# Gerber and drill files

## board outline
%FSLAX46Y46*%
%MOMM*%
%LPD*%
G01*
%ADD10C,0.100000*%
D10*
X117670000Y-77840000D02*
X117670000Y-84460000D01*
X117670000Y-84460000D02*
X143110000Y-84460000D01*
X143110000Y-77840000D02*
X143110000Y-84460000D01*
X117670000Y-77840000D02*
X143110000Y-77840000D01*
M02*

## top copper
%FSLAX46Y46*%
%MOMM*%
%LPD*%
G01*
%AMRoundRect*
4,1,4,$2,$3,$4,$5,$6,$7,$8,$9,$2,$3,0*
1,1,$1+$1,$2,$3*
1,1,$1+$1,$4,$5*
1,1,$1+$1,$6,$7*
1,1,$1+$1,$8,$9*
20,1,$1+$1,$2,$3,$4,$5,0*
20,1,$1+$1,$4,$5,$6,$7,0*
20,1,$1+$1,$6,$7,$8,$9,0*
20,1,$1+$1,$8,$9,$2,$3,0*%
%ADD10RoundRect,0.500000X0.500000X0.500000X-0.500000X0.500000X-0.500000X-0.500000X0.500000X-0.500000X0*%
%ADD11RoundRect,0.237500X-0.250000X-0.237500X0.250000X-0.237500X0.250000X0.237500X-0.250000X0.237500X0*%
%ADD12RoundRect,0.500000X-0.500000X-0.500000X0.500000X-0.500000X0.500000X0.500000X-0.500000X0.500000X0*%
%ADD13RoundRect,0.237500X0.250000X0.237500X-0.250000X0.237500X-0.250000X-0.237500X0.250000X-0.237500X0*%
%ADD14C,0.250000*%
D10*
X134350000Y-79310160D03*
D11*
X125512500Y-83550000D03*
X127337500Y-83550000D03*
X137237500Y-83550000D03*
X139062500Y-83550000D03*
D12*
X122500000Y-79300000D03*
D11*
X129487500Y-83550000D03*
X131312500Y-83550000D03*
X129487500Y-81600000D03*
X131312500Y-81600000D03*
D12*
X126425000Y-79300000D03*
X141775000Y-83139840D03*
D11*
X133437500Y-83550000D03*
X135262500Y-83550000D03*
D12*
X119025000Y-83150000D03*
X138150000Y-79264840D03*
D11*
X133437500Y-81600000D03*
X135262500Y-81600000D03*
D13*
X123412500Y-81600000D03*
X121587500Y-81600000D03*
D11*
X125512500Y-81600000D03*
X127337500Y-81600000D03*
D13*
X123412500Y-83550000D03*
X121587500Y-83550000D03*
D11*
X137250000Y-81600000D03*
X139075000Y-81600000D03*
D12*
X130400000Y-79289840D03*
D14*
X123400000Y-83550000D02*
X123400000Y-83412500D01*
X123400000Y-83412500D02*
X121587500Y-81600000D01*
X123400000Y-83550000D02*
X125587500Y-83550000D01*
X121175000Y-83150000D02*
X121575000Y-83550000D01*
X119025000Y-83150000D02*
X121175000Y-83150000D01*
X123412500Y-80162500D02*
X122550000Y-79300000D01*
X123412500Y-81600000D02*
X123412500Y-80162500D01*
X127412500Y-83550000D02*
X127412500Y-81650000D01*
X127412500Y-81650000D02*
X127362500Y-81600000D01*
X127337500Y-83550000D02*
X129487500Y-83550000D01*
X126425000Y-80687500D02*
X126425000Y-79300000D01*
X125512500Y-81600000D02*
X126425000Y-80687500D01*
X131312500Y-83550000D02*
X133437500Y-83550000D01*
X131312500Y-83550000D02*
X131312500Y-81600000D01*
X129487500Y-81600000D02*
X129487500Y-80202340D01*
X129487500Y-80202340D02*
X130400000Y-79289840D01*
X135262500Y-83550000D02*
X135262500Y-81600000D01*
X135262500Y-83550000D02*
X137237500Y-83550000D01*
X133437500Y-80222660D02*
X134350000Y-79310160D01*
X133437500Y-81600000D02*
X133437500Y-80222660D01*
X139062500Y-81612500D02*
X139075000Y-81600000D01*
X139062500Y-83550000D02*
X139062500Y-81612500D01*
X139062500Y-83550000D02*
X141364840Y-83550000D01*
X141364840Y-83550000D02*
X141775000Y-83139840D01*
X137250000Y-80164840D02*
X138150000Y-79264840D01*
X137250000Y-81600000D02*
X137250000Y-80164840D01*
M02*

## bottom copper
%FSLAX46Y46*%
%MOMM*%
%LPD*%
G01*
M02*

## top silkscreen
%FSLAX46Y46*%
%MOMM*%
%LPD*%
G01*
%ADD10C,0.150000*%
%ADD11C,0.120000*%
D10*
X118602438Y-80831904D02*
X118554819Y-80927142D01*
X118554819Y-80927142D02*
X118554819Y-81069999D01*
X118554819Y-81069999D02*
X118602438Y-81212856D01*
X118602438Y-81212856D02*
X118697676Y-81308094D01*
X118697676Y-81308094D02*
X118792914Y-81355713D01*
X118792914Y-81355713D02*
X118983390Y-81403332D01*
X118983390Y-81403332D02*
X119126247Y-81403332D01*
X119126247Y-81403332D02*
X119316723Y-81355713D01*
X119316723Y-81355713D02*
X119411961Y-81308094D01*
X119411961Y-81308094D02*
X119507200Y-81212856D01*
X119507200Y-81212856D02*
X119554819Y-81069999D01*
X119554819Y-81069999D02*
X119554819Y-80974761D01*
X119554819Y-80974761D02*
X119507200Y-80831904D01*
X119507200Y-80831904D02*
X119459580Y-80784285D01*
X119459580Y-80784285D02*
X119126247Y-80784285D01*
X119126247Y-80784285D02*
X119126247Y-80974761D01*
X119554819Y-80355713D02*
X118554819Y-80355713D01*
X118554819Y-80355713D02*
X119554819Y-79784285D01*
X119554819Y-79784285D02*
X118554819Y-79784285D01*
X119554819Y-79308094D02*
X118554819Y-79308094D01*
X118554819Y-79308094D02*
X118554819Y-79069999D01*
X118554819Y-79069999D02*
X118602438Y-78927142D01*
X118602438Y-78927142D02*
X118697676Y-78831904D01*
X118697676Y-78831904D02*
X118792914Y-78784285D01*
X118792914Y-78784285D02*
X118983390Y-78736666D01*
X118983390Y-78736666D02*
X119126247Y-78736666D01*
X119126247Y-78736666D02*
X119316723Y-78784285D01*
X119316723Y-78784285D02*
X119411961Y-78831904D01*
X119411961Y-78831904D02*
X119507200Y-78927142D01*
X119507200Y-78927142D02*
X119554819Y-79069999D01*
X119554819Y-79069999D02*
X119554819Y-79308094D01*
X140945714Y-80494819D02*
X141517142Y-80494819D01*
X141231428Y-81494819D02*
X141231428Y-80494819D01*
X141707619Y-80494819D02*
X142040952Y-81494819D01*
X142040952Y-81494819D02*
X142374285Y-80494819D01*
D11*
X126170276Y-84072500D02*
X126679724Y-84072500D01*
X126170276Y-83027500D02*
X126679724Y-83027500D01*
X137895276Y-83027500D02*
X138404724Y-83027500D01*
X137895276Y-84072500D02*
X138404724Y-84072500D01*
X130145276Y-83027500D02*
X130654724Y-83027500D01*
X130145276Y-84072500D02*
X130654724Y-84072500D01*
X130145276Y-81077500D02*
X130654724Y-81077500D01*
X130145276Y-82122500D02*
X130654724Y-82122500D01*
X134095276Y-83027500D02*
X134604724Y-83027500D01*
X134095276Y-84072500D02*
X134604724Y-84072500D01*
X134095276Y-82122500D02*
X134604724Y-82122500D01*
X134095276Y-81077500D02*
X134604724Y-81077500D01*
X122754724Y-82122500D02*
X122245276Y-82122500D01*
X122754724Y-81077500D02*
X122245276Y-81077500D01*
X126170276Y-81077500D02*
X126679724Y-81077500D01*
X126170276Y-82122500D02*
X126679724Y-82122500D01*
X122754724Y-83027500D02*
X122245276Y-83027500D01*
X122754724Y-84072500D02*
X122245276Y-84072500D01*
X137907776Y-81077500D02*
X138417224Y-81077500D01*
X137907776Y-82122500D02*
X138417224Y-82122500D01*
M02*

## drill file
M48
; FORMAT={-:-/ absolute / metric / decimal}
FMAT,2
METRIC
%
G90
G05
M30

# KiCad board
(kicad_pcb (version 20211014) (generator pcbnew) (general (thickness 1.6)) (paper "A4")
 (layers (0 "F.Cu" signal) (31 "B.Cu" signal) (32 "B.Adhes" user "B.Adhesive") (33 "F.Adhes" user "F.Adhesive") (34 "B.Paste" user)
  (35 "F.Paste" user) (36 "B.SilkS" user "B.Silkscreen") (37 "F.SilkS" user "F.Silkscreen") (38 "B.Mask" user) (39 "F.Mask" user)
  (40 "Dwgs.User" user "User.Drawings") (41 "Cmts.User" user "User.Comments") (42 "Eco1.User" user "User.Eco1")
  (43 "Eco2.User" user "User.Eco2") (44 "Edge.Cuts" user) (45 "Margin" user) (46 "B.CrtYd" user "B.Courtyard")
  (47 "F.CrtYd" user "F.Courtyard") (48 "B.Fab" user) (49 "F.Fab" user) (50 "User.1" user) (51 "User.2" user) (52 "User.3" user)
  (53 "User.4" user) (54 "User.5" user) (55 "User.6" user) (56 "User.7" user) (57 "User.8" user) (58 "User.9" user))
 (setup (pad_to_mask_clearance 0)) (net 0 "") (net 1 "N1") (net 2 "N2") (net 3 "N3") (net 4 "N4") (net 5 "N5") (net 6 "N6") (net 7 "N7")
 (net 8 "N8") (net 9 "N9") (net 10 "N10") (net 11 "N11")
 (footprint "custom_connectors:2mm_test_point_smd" (layer "F.Cu") (at 134.35 79.3 180)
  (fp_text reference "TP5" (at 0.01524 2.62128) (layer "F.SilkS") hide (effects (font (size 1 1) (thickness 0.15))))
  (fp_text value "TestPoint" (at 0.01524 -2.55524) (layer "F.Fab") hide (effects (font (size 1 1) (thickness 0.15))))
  (pad "1" smd roundrect locked (at 0 -0.01016 180) (size 2 2) (layers "F.Cu" "F.Paste" "F.Mask") (roundrect_rratio 0.25) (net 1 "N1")))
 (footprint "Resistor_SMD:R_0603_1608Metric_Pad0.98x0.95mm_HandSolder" (layer "F.Cu") (at 126.425 83.55)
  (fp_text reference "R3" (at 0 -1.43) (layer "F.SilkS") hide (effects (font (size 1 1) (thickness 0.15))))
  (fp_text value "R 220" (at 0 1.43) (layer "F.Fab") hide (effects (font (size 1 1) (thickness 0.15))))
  (fp_line (start -0.254724 0.5225) (end 0.254724 0.5225) (layer "F.SilkS") (width 0.12))
  (fp_line (start -0.254724 -0.5225) (end 0.254724 -0.5225) (layer "F.SilkS") (width 0.12))
  (pad "1" smd roundrect (at -0.9125 0) (size 0.975 0.95) (layers "F.Cu" "F.Paste" "F.Mask") (roundrect_rratio 0.25) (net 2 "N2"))
  (pad "2" smd roundrect (at 0.9125 0) (size 0.975 0.95) (layers "F.Cu" "F.Paste" "F.Mask") (roundrect_rratio 0.25) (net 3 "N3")))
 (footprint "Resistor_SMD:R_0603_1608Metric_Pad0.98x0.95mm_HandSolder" (layer "F.Cu") (at 138.15 83.55)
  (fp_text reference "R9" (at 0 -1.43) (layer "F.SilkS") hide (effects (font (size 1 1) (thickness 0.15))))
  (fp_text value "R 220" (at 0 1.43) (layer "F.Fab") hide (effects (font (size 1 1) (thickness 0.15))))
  (fp_line (start -0.254724 -0.5225) (end 0.254724 -0.5225) (layer "F.SilkS") (width 0.12))
  (fp_line (start -0.254724 0.5225) (end 0.254724 0.5225) (layer "F.SilkS") (width 0.12))
  (pad "1" smd roundrect (at -0.9125 0) (size 0.975 0.95) (layers "F.Cu" "F.Paste" "F.Mask") (roundrect_rratio 0.25) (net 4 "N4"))
  (pad "2" smd roundrect (at 0.9125 0) (size 0.975 0.95) (layers "F.Cu" "F.Paste" "F.Mask") (roundrect_rratio 0.25) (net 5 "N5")))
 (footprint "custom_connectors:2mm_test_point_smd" (layer "F.Cu") (at 122.5 79.31016)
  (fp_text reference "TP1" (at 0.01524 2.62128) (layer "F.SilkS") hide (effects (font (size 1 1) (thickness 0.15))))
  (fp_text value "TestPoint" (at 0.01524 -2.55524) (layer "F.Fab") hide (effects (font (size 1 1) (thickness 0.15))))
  (pad "1" smd roundrect locked (at 0 -0.01016) (size 2 2) (layers "F.Cu" "F.Paste" "F.Mask") (roundrect_rratio 0.25) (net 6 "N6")))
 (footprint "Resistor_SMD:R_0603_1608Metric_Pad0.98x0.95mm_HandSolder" (layer "F.Cu") (at 130.4 83.55)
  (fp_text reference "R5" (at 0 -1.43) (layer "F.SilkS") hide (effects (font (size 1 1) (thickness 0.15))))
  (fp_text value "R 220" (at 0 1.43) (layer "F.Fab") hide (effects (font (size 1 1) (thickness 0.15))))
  (fp_line (start -0.254724 -0.5225) (end 0.254724 -0.5225) (layer "F.SilkS") (width 0.12))
  (fp_line (start -0.254724 0.5225) (end 0.254724 0.5225) (layer "F.SilkS") (width 0.12))
  (pad "1" smd roundrect (at -0.9125 0) (size 0.975 0.95) (layers "F.Cu" "F.Paste" "F.Mask") (roundrect_rratio 0.25) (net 3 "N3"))
  (pad "2" smd roundrect (at 0.9125 0) (size 0.975 0.95) (layers "F.Cu" "F.Paste" "F.Mask") (roundrect_rratio 0.25) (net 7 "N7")))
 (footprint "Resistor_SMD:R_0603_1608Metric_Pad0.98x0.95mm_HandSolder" (layer "F.Cu") (at 130.4 81.6)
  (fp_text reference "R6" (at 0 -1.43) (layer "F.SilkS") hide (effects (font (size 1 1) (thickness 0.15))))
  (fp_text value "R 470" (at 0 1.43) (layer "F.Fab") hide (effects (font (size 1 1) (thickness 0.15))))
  (fp_line (start -0.254724 -0.5225) (end 0.254724 -0.5225) (layer "F.SilkS") (width 0.12))
  (fp_line (start -0.254724 0.5225) (end 0.254724 0.5225) (layer "F.SilkS") (width 0.12))
  (pad "1" smd roundrect (at -0.9125 0) (size 0.975 0.95) (layers "F.Cu" "F.Paste" "F.Mask") (roundrect_rratio 0.25) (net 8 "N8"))
  (pad "2" smd roundrect (at 0.9125 0) (size 0.975 0.95) (layers "F.Cu" "F.Paste" "F.Mask") (roundrect_rratio 0.25) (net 7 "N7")))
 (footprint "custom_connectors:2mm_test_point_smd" (layer "F.Cu") (at 126.425 79.31016)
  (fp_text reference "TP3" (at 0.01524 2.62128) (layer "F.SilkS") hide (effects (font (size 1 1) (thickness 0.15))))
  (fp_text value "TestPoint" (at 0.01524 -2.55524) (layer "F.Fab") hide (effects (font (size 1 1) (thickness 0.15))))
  (pad "1" smd roundrect locked (at 0 -0.01016) (size 2 2) (layers "F.Cu" "F.Paste" "F.Mask") (roundrect_rratio 0.25) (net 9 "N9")))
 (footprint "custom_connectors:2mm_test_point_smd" (layer "F.Cu") (at 141.775 83.15)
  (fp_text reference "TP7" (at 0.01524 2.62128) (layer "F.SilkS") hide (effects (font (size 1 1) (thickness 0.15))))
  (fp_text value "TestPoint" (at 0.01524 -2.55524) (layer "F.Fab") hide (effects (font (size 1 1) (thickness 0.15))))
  (pad "1" smd roundrect locked (at 0 -0.01016) (size 2 2) (layers "F.Cu" "F.Paste" "F.Mask") (roundrect_rratio 0.25) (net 5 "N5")))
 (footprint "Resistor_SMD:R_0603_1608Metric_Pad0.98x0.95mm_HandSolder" (layer "F.Cu") (at 134.35 83.55)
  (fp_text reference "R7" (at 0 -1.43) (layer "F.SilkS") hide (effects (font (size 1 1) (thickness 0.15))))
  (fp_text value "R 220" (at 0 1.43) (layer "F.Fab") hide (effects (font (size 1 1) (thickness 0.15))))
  (fp_line (start -0.254724 -0.5225) (end 0.254724 -0.5225) (layer "F.SilkS") (width 0.12))
  (fp_line (start -0.254724 0.5225) (end 0.254724 0.5225) (layer "F.SilkS") (width 0.12))
  (pad "1" smd roundrect (at -0.9125 0) (size 0.975 0.95) (layers "F.Cu" "F.Paste" "F.Mask") (roundrect_rratio 0.25) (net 7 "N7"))
  (pad "2" smd roundrect (at 0.9125 0) (size 0.975 0.95) (layers "F.Cu" "F.Paste" "F.Mask") (roundrect_rratio 0.25) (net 4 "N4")))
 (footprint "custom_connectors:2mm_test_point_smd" (layer "F.Cu") (at 119.025 83.16016)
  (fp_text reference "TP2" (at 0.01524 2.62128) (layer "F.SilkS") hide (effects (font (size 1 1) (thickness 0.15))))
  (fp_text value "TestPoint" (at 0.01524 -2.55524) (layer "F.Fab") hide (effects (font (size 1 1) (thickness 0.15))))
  (pad "1" smd roundrect locked (at 0 -0.01016) (size 2 2) (layers "F.Cu" "F.Paste" "F.Mask") (roundrect_rratio 0.25) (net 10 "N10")))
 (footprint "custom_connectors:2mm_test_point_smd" (layer "F.Cu") (at 138.15 79.275)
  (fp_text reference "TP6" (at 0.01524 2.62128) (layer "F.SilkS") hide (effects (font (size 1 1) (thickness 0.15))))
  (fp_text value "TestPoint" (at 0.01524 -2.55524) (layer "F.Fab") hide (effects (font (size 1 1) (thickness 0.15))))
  (pad "1" smd roundrect locked (at 0 -0.01016) (size 2 2) (layers "F.Cu" "F.Paste" "F.Mask") (roundrect_rratio 0.25) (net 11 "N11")))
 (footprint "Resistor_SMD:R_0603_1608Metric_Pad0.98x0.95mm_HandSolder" (layer "F.Cu") (at 134.35 81.6)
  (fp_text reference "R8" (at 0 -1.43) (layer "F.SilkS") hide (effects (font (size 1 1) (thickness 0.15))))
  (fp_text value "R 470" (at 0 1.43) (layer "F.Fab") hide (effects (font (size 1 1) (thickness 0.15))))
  (fp_line (start -0.254724 0.5225) (end 0.254724 0.5225) (layer "F.SilkS") (width 0.12))
  (fp_line (start -0.254724 -0.5225) (end 0.254724 -0.5225) (layer "F.SilkS") (width 0.12))
  (pad "1" smd roundrect (at -0.9125 0) (size 0.975 0.95) (layers "F.Cu" "F.Paste" "F.Mask") (roundrect_rratio 0.25) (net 1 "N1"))
  (pad "2" smd roundrect (at 0.9125 0) (size 0.975 0.95) (layers "F.Cu" "F.Paste" "F.Mask") (roundrect_rratio 0.25) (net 4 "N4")))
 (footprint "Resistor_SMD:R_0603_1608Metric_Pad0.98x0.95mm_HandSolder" (layer "F.Cu") (at 122.5 81.6 180)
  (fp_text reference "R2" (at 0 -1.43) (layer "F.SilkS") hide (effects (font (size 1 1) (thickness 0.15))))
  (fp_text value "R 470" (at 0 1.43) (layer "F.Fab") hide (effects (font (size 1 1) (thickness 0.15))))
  (fp_line (start -0.254724 -0.5225) (end 0.254724 -0.5225) (layer "F.SilkS") (width 0.12))
  (fp_line (start -0.254724 0.5225) (end 0.254724 0.5225) (layer "F.SilkS") (width 0.12))
  (pad "1" smd roundrect (at -0.9125 0 180) (size 0.975 0.95) (layers "F.Cu" "F.Paste" "F.Mask") (roundrect_rratio 0.25) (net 6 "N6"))
  (pad "2" smd roundrect (at 0.9125 0 180) (size 0.975 0.95) (layers "F.Cu" "F.Paste" "F.Mask") (roundrect_rratio 0.25) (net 2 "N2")))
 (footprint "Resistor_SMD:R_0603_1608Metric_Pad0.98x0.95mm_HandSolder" (layer "F.Cu") (at 126.425 81.6)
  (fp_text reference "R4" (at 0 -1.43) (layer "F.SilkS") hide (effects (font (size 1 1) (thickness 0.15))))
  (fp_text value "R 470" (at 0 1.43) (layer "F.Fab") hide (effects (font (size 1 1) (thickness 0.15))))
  (fp_line (start -0.254724 -0.5225) (end 0.254724 -0.5225) (layer "F.SilkS") (width 0.12))
  (fp_line (start -0.254724 0.5225) (end 0.254724 0.5225) (layer "F.SilkS") (width 0.12))
  (pad "1" smd roundrect (at -0.9125 0) (size 0.975 0.95) (layers "F.Cu" "F.Paste" "F.Mask") (roundrect_rratio 0.25) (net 9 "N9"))
  (pad "2" smd roundrect (at 0.9125 0) (size 0.975 0.95) (layers "F.Cu" "F.Paste" "F.Mask") (roundrect_rratio 0.25) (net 3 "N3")))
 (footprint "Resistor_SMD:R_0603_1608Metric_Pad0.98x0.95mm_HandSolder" (layer "F.Cu") (at 122.5 83.55 180)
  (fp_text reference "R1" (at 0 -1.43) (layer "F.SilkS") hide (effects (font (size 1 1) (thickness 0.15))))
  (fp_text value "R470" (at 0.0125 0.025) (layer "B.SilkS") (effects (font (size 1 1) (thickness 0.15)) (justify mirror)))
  (fp_line (start -0.254724 0.5225) (end 0.254724 0.5225) (layer "F.SilkS") (width 0.12))
  (fp_line (start -0.254724 -0.5225) (end 0.254724 -0.5225) (layer "F.SilkS") (width 0.12))
  (pad "1" smd roundrect (at -0.9125 0 180) (size 0.975 0.95) (layers "F.Cu" "F.Paste" "F.Mask") (roundrect_rratio 0.25) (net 2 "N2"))
  (pad "2" smd roundrect (at 0.9125 0 180) (size 0.975 0.95) (layers "F.Cu" "F.Paste" "F.Mask") (roundrect_rratio 0.25) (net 10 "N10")))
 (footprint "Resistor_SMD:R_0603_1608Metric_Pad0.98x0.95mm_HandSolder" (layer "F.Cu") (at 138.1625 81.6)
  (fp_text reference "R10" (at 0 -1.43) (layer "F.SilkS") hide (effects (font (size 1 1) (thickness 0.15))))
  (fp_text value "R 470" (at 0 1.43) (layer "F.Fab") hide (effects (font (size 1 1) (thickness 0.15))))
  (fp_line (start -0.254724 -0.5225) (end 0.254724 -0.5225) (layer "F.SilkS") (width 0.12))
  (fp_line (start -0.254724 0.5225) (end 0.254724 0.5225) (layer "F.SilkS") (width 0.12))
  (pad "1" smd roundrect (at -0.9125 0) (size 0.975 0.95) (layers "F.Cu" "F.Paste" "F.Mask") (roundrect_rratio 0.25) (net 11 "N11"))
  (pad "2" smd roundrect (at 0.9125 0) (size 0.975 0.95) (layers "F.Cu" "F.Paste" "F.Mask") (roundrect_rratio 0.25) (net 5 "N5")))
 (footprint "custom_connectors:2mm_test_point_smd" (layer "F.Cu") (at 130.4 79.3)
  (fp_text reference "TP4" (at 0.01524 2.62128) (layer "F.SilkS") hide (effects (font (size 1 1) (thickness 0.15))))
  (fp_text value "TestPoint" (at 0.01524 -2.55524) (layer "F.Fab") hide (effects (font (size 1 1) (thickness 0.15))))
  (pad "1" smd roundrect locked (at 0 -0.01016) (size 2 2) (layers "F.Cu" "F.Paste" "F.Mask") (roundrect_rratio 0.25) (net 8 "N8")))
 (gr_line (start 117.67 77.84) (end 117.67 84.46) (layer "Edge.Cuts") (width 0.1))
 (gr_line (start 117.67 84.46) (end 143.11 84.46) (layer "Edge.Cuts") (width 0.1))
 (gr_line (start 143.11 77.84) (end 143.11 84.46) (layer "Edge.Cuts") (width 0.1))
 (gr_line (start 117.67 77.84) (end 143.11 77.84) (layer "Edge.Cuts") (width 0.1))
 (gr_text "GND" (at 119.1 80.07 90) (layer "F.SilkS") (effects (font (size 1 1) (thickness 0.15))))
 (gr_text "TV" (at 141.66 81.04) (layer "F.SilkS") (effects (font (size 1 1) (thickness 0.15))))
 (segment (start 123.4 83.55) (end 123.4 83.4125) (width 0.25) (layer "F.Cu") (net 2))
 (segment (start 123.4 83.4125) (end 121.5875 81.6) (width 0.25) (layer "F.Cu") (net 2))
 (segment (start 123.4 83.55) (end 125.5875 83.55) (width 0.25) (layer "F.Cu") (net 2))
 (segment (start 121.175 83.15) (end 121.575 83.55) (width 0.25) (layer "F.Cu") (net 10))
 (segment (start 119.025 83.15) (end 121.175 83.15) (width 0.25) (layer "F.Cu") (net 10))
 (segment (start 123.4125 80.1625) (end 122.55 79.3) (width 0.25) (layer "F.Cu") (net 6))
 (segment (start 123.4125 81.6) (end 123.4125 80.1625) (width 0.25) (layer "F.Cu") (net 6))
 (segment (start 127.4125 83.55) (end 127.4125 81.65) (width 0.25) (layer "F.Cu") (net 3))
 (segment (start 127.4125 81.65) (end 127.3625 81.6) (width 0.25) (layer "F.Cu") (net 3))
 (segment (start 127.3375 83.55) (end 129.4875 83.55) (width 0.25) (layer "F.Cu") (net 3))
 (segment (start 126.425 80.6875) (end 126.425 79.3) (width 0.25) (layer "F.Cu") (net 9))
 (segment (start 125.5125 81.6) (end 126.425 80.6875) (width 0.25) (layer "F.Cu") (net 9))
 (segment (start 131.3125 83.55) (end 133.4375 83.55) (width 0.25) (layer "F.Cu") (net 7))
 (segment (start 131.3125 83.55) (end 131.3125 81.6) (width 0.25) (layer "F.Cu") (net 7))
 (segment (start 129.4875 81.6) (end 129.4875 80.20234) (width 0.25) (layer "F.Cu") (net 8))
 (segment (start 129.4875 80.20234) (end 130.4 79.28984) (width 0.25) (layer "F.Cu") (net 8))
 (segment (start 135.2625 83.55) (end 135.2625 81.6) (width 0.25) (layer "F.Cu") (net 4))
 (segment (start 135.2625 83.55) (end 137.2375 83.55) (width 0.25) (layer "F.Cu") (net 4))
 (segment (start 133.4375 80.22266) (end 134.35 79.31016) (width 0.25) (layer "F.Cu") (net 1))
 (segment (start 133.4375 81.6) (end 133.4375 80.22266) (width 0.25) (layer "F.Cu") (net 1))
 (segment (start 139.0625 81.6125) (end 139.075 81.6) (width 0.25) (layer "F.Cu") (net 5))
 (segment (start 139.0625 83.55) (end 139.0625 81.6125) (width 0.25) (layer "F.Cu") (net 5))
 (segment (start 139.0625 83.55) (end 141.36484 83.55) (width 0.25) (layer "F.Cu") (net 5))
 (segment (start 141.36484 83.55) (end 141.775 83.13984) (width 0.25) (layer "F.Cu") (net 5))
 (segment (start 137.25 80.16484) (end 138.15 79.26484) (width 0.25) (layer "F.Cu") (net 11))
 (segment (start 137.25 81.6) (end 137.25 80.16484) (width 0.25) (layer "F.Cu") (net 11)))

